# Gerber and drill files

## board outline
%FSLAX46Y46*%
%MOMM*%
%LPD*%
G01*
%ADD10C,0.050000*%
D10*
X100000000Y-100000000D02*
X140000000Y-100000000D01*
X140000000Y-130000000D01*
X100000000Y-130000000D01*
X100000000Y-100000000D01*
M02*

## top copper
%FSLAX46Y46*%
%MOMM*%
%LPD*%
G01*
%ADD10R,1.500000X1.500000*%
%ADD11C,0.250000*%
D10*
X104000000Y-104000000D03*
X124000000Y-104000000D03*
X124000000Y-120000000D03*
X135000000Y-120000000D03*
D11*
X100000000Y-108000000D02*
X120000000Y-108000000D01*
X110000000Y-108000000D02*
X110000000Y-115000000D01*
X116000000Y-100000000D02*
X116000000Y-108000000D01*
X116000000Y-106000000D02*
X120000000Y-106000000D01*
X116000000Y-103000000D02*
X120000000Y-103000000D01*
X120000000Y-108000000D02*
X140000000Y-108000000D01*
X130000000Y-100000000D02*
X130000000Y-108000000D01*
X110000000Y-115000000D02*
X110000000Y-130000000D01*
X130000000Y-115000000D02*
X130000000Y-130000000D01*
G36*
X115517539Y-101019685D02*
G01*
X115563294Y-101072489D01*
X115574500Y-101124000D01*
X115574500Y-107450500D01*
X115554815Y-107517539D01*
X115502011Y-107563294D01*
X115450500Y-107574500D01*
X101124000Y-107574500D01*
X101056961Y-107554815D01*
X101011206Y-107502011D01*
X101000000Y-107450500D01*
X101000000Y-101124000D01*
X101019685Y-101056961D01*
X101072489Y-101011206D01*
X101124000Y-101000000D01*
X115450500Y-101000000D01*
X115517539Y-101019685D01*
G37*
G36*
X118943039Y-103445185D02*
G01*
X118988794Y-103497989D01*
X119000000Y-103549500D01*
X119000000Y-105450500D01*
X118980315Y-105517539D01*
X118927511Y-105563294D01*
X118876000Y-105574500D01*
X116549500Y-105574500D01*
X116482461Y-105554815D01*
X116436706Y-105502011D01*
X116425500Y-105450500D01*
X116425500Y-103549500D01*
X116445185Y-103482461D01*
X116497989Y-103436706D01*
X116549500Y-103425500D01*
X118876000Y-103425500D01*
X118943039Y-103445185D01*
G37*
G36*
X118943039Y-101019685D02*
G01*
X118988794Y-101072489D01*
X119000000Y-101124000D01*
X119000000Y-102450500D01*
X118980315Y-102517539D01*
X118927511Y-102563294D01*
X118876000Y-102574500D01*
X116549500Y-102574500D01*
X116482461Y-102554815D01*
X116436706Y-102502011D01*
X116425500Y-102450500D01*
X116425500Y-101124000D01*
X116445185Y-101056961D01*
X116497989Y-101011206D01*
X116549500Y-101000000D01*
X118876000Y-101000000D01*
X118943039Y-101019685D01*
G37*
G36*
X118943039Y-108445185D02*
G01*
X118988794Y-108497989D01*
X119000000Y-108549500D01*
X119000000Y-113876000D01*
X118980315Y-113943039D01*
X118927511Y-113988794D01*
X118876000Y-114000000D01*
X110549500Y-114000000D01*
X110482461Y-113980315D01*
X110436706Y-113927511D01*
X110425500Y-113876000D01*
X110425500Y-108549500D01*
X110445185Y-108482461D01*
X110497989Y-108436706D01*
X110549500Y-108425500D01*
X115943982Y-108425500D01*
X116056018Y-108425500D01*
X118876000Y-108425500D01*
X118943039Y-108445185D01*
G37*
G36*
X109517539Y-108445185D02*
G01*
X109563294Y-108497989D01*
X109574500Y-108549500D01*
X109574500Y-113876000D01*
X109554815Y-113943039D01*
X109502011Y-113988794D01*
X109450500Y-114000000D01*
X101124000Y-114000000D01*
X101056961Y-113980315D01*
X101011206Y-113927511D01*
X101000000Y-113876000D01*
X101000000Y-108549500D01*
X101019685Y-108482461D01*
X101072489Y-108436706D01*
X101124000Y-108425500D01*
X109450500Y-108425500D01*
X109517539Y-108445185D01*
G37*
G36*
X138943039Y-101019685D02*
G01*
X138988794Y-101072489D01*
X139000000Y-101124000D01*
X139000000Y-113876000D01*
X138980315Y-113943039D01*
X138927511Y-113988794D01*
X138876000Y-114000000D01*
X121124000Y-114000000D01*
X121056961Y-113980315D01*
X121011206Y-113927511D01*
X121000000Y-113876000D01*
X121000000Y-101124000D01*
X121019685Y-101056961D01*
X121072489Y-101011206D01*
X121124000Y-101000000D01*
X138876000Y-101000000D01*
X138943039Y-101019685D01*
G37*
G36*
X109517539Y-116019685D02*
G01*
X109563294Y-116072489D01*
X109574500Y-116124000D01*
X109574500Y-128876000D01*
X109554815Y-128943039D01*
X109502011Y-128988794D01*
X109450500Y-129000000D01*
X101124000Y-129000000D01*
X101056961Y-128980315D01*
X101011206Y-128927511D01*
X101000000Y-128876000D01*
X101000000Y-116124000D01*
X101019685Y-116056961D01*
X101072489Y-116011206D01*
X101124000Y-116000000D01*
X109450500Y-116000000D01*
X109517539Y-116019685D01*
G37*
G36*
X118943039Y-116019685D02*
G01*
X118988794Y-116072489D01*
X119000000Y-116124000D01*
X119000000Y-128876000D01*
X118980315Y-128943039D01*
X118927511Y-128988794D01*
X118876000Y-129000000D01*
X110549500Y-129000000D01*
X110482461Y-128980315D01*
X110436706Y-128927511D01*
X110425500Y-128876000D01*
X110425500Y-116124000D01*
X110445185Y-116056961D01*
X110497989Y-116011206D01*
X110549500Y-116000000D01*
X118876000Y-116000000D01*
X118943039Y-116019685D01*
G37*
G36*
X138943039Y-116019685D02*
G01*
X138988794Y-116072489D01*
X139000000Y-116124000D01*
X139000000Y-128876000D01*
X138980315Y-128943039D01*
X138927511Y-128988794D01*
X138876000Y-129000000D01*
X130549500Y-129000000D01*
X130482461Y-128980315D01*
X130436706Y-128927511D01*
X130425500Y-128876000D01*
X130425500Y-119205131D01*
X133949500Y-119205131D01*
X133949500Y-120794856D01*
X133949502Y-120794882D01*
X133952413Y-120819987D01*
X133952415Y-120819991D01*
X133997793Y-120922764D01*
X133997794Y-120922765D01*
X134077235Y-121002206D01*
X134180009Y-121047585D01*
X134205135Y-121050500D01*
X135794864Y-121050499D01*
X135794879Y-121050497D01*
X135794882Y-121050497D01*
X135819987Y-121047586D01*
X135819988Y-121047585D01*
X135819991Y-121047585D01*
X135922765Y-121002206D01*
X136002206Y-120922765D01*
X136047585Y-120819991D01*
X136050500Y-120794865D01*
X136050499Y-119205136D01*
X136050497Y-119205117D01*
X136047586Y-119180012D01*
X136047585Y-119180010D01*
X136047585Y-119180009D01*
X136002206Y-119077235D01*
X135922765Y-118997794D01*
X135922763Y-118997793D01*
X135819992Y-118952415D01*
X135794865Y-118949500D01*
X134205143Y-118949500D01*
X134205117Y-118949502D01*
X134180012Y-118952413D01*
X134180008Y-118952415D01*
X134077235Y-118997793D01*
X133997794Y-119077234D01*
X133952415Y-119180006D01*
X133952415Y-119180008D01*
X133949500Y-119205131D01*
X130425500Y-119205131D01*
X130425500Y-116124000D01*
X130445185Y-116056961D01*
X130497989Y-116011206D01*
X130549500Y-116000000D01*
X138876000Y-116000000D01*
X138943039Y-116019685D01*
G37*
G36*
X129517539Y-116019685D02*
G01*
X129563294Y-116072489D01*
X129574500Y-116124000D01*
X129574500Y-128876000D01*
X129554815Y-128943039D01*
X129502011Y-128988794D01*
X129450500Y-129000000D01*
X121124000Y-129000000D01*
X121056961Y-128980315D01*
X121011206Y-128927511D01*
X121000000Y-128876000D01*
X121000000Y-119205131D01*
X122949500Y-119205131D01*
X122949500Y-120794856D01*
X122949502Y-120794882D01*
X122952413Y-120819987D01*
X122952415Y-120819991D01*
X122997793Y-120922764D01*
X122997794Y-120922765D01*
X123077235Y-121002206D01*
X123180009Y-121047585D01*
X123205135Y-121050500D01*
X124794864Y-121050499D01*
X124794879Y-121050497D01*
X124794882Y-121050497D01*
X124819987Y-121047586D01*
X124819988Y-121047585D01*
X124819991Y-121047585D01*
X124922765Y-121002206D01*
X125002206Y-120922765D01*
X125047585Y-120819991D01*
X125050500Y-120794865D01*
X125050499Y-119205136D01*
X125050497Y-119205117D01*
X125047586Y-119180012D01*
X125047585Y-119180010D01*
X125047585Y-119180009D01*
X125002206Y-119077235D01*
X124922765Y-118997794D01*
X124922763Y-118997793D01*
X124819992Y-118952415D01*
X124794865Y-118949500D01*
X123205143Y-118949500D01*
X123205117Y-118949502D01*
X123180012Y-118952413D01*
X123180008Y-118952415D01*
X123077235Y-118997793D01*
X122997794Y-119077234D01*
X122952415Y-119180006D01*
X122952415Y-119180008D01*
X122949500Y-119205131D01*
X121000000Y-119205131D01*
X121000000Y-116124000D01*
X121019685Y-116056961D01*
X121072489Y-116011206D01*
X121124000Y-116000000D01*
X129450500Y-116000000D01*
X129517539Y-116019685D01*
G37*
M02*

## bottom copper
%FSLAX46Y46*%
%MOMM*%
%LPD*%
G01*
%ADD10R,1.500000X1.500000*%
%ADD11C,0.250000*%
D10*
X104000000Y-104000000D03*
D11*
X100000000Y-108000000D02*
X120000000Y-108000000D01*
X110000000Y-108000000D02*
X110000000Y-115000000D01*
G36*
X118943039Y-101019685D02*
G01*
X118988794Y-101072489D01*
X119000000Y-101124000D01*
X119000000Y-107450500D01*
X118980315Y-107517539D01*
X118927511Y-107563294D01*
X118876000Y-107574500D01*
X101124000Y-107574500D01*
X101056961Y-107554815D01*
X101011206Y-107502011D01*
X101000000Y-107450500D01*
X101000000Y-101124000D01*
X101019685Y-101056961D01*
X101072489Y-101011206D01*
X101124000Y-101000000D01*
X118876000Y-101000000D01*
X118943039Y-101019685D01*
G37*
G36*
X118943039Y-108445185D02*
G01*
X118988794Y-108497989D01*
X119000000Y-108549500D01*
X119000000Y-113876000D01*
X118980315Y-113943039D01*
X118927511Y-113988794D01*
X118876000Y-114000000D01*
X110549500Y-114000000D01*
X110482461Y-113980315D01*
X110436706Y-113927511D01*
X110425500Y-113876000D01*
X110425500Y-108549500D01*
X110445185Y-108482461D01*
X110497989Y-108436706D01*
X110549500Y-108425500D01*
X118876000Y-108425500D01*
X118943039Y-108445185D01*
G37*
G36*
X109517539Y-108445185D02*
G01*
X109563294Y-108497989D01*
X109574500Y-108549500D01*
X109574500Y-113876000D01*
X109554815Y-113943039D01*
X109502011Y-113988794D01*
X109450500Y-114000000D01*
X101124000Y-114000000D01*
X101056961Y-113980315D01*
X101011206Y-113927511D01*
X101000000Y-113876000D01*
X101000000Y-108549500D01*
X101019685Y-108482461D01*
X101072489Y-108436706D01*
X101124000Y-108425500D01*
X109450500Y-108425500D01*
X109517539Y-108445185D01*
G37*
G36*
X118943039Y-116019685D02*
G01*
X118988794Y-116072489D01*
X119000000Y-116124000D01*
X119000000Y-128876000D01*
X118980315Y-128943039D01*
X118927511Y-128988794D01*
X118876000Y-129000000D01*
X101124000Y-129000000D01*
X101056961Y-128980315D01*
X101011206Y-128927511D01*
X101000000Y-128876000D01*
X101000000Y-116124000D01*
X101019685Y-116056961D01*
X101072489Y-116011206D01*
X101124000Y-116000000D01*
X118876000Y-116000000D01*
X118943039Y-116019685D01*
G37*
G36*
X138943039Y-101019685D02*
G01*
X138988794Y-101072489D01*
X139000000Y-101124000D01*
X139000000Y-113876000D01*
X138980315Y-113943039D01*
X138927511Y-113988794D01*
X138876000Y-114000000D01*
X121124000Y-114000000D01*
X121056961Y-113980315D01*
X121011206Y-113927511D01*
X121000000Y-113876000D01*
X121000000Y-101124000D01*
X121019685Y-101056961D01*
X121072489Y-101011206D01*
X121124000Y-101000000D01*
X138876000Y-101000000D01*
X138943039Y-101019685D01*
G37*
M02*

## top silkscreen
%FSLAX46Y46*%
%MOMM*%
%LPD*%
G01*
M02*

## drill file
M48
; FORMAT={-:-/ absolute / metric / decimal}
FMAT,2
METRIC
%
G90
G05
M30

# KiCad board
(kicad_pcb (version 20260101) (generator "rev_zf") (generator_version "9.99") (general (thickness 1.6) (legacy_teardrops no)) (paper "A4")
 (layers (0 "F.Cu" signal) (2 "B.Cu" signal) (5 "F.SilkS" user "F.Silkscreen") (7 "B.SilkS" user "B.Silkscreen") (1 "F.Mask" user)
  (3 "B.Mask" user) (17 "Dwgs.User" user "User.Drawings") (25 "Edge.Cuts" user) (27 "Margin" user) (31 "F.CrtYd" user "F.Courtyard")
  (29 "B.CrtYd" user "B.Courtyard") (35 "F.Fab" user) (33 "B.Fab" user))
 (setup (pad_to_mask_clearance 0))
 (gr_rect (start 100.0 100.0) (end 140.0 130.0) (stroke (width 0.05) (type default)) (fill no) (layer "Edge.Cuts"))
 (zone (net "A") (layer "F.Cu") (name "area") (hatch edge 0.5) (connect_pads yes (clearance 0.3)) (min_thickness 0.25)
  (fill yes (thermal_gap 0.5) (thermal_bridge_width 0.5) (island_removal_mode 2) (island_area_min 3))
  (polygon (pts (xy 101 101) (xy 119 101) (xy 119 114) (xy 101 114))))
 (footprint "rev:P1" (layer "F.Cu") (at 104 104)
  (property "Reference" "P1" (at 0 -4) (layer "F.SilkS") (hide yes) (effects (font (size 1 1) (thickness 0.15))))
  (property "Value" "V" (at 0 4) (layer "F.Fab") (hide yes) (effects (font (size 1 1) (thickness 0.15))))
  (pad "1" smd rect (at 0 0) (size 1.5 1.5) (layers "F.Cu" "F.Mask") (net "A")))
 (segment (start 100 108) (end 120 108) (width 0.25) (layer "F.Cu") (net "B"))
 (segment (start 110 108) (end 110 115) (width 0.25) (layer "F.Cu") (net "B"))
 (segment (start 116 100) (end 116 108) (width 0.25) (layer "F.Cu") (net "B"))
 (segment (start 116 106) (end 120 106) (width 0.25) (layer "F.Cu") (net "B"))
 (segment (start 116 103) (end 120 103) (width 0.25) (layer "F.Cu") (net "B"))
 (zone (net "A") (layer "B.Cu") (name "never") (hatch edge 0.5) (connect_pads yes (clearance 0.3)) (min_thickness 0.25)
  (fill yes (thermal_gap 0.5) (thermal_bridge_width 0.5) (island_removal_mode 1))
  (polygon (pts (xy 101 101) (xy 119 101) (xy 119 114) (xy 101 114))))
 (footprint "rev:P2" (layer "B.Cu") (at 104 104)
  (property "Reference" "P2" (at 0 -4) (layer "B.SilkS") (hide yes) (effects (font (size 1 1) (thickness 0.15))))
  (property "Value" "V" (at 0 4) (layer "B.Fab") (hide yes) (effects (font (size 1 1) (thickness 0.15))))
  (pad "1" smd rect (at 0 0) (size 1.5 1.5) (layers "B.Cu" "B.Mask") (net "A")))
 (segment (start 100 108) (end 120 108) (width 0.25) (layer "B.Cu") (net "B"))
 (segment (start 110 108) (end 110 115) (width 0.25) (layer "B.Cu") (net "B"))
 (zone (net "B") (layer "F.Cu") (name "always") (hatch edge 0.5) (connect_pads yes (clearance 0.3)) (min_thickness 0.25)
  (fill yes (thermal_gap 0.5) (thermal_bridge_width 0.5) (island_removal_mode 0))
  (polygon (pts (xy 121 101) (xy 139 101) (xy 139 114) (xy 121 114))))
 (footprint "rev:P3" (layer "F.Cu") (at 124 104)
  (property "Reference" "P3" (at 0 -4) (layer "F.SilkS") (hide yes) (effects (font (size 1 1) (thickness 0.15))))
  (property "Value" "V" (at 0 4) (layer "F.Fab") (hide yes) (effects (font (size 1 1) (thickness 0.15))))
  (pad "1" smd rect (at 0 0) (size 1.5 1.5) (layers "F.Cu" "F.Mask") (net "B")))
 (segment (start 120 108) (end 140 108) (width 0.25) (layer "F.Cu") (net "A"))
 (segment (start 130 100) (end 130 108) (width 0.25) (layer "F.Cu") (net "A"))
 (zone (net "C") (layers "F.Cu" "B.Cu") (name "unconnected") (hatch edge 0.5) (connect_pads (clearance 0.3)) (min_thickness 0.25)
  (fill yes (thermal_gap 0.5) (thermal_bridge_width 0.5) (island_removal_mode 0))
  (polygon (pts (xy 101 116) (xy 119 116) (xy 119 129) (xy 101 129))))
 (segment (start 110 115) (end 110 130) (width 0.25) (layer "F.Cu") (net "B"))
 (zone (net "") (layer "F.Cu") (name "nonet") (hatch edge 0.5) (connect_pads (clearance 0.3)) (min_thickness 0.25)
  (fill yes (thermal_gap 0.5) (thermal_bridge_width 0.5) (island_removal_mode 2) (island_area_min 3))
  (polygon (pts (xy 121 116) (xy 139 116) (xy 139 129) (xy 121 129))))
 (segment (start 130 115) (end 130 130) (width 0.25) (layer "F.Cu") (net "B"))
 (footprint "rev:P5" (layer "F.Cu") (at 124 120)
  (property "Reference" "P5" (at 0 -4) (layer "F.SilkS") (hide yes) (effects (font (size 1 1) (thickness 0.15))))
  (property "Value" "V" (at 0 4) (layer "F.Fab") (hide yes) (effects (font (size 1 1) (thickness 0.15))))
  (pad "1" smd rect (at 0 0) (size 1.5 1.5) (layers "F.Cu" "F.Mask") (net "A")))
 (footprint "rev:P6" (layer "F.Cu") (at 135 120)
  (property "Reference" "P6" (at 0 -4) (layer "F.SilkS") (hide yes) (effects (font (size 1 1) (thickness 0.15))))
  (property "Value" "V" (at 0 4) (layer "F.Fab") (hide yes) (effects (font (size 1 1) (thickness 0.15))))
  (pad "1" smd rect (at 0 0) (size 1.5 1.5) (layers "F.Cu" "F.Mask")))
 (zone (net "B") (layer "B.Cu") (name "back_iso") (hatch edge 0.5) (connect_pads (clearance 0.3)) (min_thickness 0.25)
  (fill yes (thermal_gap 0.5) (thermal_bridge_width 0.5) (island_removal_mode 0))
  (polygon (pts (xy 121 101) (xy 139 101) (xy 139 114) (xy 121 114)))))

